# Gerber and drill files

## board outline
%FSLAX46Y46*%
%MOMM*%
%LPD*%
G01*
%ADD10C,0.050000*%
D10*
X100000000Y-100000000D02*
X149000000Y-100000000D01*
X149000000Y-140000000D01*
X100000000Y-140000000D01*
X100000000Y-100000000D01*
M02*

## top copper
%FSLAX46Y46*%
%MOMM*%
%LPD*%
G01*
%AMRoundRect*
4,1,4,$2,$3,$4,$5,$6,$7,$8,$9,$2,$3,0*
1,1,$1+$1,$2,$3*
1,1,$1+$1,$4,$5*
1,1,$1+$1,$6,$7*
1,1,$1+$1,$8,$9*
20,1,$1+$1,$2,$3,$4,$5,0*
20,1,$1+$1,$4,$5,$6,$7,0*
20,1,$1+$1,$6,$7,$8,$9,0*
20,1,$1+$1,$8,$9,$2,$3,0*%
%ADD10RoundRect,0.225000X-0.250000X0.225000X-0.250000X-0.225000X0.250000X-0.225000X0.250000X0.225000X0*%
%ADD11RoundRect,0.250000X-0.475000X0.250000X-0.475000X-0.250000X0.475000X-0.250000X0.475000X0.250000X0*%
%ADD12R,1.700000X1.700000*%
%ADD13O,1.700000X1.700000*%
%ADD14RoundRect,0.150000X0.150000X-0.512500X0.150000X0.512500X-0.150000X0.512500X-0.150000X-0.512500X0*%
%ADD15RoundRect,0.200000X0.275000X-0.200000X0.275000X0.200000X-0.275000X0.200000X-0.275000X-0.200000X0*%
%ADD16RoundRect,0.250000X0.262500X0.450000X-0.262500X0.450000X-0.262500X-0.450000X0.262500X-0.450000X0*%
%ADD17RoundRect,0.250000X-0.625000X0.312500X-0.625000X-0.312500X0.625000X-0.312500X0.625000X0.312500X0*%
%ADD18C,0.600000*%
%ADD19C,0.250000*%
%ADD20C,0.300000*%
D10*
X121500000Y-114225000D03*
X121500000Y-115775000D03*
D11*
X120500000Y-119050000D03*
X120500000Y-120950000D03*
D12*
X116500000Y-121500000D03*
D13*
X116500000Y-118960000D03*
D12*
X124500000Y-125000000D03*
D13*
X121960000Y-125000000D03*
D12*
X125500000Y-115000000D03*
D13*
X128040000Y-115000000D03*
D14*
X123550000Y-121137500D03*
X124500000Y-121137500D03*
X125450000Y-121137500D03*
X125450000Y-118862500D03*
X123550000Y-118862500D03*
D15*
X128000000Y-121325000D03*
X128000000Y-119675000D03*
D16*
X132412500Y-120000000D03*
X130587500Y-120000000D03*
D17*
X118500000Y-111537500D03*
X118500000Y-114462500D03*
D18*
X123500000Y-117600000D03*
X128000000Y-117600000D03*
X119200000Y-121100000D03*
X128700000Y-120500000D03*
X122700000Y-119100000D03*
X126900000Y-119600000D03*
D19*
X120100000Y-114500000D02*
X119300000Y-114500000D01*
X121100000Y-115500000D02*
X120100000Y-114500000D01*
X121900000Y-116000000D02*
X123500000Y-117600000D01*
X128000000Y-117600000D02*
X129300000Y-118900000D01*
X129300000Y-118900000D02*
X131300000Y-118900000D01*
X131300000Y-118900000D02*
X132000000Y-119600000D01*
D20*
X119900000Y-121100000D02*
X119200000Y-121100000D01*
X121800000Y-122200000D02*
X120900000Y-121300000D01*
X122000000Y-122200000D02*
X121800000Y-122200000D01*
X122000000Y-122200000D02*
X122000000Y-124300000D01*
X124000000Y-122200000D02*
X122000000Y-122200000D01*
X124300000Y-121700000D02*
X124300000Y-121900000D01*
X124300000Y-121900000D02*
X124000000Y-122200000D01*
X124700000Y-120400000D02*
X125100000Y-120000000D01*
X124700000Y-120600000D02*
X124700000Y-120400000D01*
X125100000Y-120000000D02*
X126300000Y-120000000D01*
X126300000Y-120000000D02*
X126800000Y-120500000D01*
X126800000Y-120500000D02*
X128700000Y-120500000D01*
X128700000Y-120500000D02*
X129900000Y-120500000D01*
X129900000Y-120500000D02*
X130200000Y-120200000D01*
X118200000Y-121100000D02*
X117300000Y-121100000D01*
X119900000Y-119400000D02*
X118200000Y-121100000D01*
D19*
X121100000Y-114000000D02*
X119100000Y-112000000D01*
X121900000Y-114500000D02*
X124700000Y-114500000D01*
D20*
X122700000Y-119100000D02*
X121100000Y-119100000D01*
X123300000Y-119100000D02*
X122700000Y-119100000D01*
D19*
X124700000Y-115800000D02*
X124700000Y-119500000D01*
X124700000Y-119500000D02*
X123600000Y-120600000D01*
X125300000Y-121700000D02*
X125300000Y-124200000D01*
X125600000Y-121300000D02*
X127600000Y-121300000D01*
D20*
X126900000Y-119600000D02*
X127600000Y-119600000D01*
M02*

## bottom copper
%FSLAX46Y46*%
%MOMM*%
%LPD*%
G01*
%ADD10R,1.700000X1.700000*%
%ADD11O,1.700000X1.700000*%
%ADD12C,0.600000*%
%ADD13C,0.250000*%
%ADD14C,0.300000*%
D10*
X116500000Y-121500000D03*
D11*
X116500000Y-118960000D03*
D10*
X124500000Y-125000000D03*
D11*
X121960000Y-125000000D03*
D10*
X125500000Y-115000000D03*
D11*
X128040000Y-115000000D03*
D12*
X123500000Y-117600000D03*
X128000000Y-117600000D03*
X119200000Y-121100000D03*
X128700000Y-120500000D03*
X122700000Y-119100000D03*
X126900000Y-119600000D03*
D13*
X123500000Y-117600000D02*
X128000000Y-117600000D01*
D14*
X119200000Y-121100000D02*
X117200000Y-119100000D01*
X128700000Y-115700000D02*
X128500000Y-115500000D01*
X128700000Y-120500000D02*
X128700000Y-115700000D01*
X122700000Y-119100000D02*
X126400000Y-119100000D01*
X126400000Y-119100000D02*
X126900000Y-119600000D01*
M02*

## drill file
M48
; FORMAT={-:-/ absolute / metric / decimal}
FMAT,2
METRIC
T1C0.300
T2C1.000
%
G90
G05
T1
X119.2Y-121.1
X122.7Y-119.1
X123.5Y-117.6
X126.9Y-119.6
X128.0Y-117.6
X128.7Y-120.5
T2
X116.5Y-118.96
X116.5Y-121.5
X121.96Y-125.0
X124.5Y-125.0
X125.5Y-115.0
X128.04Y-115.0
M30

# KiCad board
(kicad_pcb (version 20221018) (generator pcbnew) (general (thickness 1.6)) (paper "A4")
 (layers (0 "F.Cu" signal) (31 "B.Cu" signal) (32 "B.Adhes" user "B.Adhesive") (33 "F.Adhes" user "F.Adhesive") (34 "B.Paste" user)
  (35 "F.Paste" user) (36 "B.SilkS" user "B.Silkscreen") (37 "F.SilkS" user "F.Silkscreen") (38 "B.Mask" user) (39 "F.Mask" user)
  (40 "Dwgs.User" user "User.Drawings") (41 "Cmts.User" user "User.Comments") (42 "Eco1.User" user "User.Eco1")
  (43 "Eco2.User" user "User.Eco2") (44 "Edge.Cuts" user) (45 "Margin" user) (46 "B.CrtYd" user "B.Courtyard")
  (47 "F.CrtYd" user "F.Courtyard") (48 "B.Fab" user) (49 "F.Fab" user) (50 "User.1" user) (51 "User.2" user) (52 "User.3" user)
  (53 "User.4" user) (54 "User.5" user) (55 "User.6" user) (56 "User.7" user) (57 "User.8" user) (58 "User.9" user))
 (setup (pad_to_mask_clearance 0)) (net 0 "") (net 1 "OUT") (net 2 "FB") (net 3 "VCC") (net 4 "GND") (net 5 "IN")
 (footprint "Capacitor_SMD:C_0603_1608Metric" (layer "F.Cu") (at 121.5 115 -90)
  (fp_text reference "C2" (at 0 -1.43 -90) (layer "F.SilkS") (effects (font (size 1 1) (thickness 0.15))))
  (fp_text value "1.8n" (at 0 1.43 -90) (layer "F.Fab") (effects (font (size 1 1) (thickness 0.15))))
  (pad "1" smd roundrect (at -0.775 0 270) (size 0.9 0.95) (layers "F.Cu" "F.Paste" "F.Mask") (roundrect_rratio 0.25) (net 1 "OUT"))
  (pad "2" smd roundrect (at 0.775 0 270) (size 0.9 0.95) (layers "F.Cu" "F.Paste" "F.Mask") (roundrect_rratio 0.25) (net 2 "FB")))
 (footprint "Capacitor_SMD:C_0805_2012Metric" (layer "F.Cu") (at 120.5 120 -90)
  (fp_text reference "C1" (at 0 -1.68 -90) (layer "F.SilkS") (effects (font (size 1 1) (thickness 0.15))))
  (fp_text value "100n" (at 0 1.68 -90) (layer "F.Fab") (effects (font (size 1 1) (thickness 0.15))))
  (pad "1" smd roundrect (at -0.95 0 270) (size 1 1.45) (layers "F.Cu" "F.Paste" "F.Mask") (roundrect_rratio 0.25) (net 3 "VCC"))
  (pad "2" smd roundrect (at 0.95 0 270) (size 1 1.45) (layers "F.Cu" "F.Paste" "F.Mask") (roundrect_rratio 0.25) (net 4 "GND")))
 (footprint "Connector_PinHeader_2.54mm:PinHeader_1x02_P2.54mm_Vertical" (layer "F.Cu") (at 116.5 121.5 180)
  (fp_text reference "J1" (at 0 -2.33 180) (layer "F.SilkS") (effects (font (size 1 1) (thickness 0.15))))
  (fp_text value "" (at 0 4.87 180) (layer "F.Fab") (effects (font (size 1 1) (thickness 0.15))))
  (pad "1" thru_hole rect (at 0 0 180) (size 1.7 1.7) (drill 1) (layers "*.Cu" "*.Mask") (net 3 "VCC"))
  (pad "2" thru_hole oval (at 0 2.54 180) (size 1.7 1.7) (drill 1) (layers "*.Cu" "*.Mask") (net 4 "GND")))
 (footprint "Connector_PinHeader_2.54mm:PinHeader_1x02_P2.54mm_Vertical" (layer "F.Cu") (at 124.5 125 -90)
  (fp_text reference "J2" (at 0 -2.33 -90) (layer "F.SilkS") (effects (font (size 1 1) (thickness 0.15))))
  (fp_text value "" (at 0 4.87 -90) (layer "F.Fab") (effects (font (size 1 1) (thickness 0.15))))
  (pad "1" thru_hole rect (at 0 0 270) (size 1.7 1.7) (drill 1) (layers "*.Cu" "*.Mask") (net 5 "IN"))
  (pad "2" thru_hole oval (at 0 2.54 270) (size 1.7 1.7) (drill 1) (layers "*.Cu" "*.Mask") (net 4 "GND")))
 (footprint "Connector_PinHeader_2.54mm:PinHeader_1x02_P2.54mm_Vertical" (layer "F.Cu") (at 125.5 115 90)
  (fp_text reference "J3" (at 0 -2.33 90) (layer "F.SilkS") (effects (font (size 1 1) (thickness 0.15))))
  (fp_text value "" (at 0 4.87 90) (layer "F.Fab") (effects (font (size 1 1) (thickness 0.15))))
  (pad "1" thru_hole rect (at 0 0 90) (size 1.7 1.7) (drill 1) (layers "*.Cu" "*.Mask") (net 1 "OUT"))
  (pad "2" thru_hole oval (at 0 2.54 90) (size 1.7 1.7) (drill 1) (layers "*.Cu" "*.Mask") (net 4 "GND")))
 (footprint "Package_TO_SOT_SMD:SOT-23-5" (layer "F.Cu") (at 124.5 120 90)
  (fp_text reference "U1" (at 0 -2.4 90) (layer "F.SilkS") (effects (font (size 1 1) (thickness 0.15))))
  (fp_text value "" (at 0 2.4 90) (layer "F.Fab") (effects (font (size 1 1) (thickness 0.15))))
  (pad "1" smd roundrect (at -1.1375 -0.95 90) (size 1.325 0.6) (layers "F.Cu" "F.Paste" "F.Mask") (roundrect_rratio 0.25) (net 1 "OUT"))
  (pad "2" smd roundrect (at -1.1375 0 90) (size 1.325 0.6) (layers "F.Cu" "F.Paste" "F.Mask") (roundrect_rratio 0.25) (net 4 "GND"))
  (pad "3" smd roundrect (at -1.1375 0.95 90) (size 1.325 0.6) (layers "F.Cu" "F.Paste" "F.Mask") (roundrect_rratio 0.25) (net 5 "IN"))
  (pad "4" smd roundrect (at 1.1375 0.95 90) (size 1.325 0.6) (layers "F.Cu" "F.Paste" "F.Mask") (roundrect_rratio 0.25))
  (pad "5" smd roundrect (at 1.1375 -0.95 90) (size 1.325 0.6) (layers "F.Cu" "F.Paste" "F.Mask") (roundrect_rratio 0.25) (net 3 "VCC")))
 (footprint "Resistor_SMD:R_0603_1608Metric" (layer "F.Cu") (at 128 120.5 90)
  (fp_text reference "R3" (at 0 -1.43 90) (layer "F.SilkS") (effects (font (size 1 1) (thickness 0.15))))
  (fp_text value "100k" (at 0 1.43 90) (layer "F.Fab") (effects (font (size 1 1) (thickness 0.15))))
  (pad "1" smd roundrect (at -0.825 0 90) (size 0.8 0.95) (layers "F.Cu" "F.Paste" "F.Mask") (roundrect_rratio 0.25) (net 5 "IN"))
  (pad "2" smd roundrect (at 0.825 0 90) (size 0.8 0.95) (layers "F.Cu" "F.Paste" "F.Mask") (roundrect_rratio 0.25) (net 3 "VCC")))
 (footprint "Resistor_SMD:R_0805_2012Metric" (layer "F.Cu") (at 131.5 120 180)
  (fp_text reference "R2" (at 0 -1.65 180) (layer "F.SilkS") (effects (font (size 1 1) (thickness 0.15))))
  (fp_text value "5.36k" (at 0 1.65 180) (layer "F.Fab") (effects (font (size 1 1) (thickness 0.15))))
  (pad "1" smd roundrect (at -0.9125 0 180) (size 1.025 1.4) (layers "F.Cu" "F.Paste" "F.Mask") (roundrect_rratio 0.243902) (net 2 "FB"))
  (pad "2" smd roundrect (at 0.9125 0 180) (size 1.025 1.4) (layers "F.Cu" "F.Paste" "F.Mask") (roundrect_rratio 0.243902) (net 4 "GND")))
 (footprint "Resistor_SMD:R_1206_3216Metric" (layer "F.Cu") (at 118.5 113 -90)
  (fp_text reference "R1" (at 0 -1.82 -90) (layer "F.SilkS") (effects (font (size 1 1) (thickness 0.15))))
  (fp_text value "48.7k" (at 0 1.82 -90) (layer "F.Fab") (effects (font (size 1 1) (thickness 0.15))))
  (pad "1" smd roundrect (at -1.4625 0 270) (size 1.125 1.75) (layers "F.Cu" "F.Paste" "F.Mask") (roundrect_rratio 0.222222) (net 1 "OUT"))
  (pad "2" smd roundrect (at 1.4625 0 270) (size 1.125 1.75) (layers "F.Cu" "F.Paste" "F.Mask") (roundrect_rratio 0.222222) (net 2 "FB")))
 (gr_rect (start 100 100) (end 149 140) (stroke (width 0.05) (type default)) (fill none) (layer "Edge.Cuts"))
 (segment (start 120.1 114.5) (end 119.3 114.5) (width 0.25) (layer "F.Cu") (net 2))
 (segment (start 121.1 115.5) (end 120.1 114.5) (width 0.25) (layer "F.Cu") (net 2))
 (segment (start 121.9 116) (end 123.5 117.6) (width 0.25) (layer "F.Cu") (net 2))
 (segment (start 128 117.6) (end 129.3 118.9) (width 0.25) (layer "F.Cu") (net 2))
 (segment (start 129.3 118.9) (end 131.3 118.9) (width 0.25) (layer "F.Cu") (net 2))
 (segment (start 131.3 118.9) (end 132 119.6) (width 0.25) (layer "F.Cu") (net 2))
 (via (at 123.5 117.6) (size 0.6) (drill 0.3) (layers "F.Cu" "B.Cu") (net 2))
 (via (at 128 117.6) (size 0.6) (drill 0.3) (layers "F.Cu" "B.Cu") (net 2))
 (segment (start 119.9 121.1) (end 119.2 121.1) (width 0.3) (layer "F.Cu") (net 4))
 (segment (start 121.8 122.2) (end 120.9 121.3) (width 0.3) (layer "F.Cu") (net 4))
 (segment (start 122 122.2) (end 121.8 122.2) (width 0.3) (layer "F.Cu") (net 4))
 (segment (start 122 122.2) (end 122 124.3) (width 0.3) (layer "F.Cu") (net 4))
 (segment (start 123.5 117.6) (end 128 117.6) (width 0.25) (layer "B.Cu") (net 2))
 (segment (start 124 122.2) (end 122 122.2) (width 0.3) (layer "F.Cu") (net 4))
 (segment (start 124.3 121.7) (end 124.3 121.9) (width 0.3) (layer "F.Cu") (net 4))
 (segment (start 124.3 121.9) (end 124 122.2) (width 0.3) (layer "F.Cu") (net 4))
 (segment (start 124.7 120.4) (end 125.1 120) (width 0.3) (layer "F.Cu") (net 4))
 (segment (start 124.7 120.6) (end 124.7 120.4) (width 0.3) (layer "F.Cu") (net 4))
 (segment (start 125.1 120) (end 126.3 120) (width 0.3) (layer "F.Cu") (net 4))
 (segment (start 126.3 120) (end 126.8 120.5) (width 0.3) (layer "F.Cu") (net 4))
 (segment (start 126.8 120.5) (end 128.7 120.5) (width 0.3) (layer "F.Cu") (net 4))
 (segment (start 128.7 120.5) (end 129.9 120.5) (width 0.3) (layer "F.Cu") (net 4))
 (segment (start 129.9 120.5) (end 130.2 120.2) (width 0.3) (layer "F.Cu") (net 4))
 (via (at 119.2 121.1) (size 0.6) (drill 0.3) (layers "F.Cu" "B.Cu") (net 4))
 (via (at 128.7 120.5) (size 0.6) (drill 0.3) (layers "F.Cu" "B.Cu") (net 4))
 (segment (start 118.2 121.1) (end 117.3 121.1) (width 0.3) (layer "F.Cu") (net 3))
 (segment (start 119.2 121.1) (end 117.2 119.1) (width 0.3) (layer "B.Cu") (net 4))
 (segment (start 119.9 119.4) (end 118.2 121.1) (width 0.3) (layer "F.Cu") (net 3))
 (segment (start 121.1 114) (end 119.1 112) (width 0.25) (layer "F.Cu") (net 1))
 (segment (start 121.9 114.5) (end 124.7 114.5) (width 0.25) (layer "F.Cu") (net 1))
 (segment (start 122.7 119.1) (end 121.1 119.1) (width 0.3) (layer "F.Cu") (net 3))
 (segment (start 123.3 119.1) (end 122.7 119.1) (width 0.3) (layer "F.Cu") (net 3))
 (segment (start 124.7 115.8) (end 124.7 119.5) (width 0.25) (layer "F.Cu") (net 1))
 (segment (start 124.7 119.5) (end 123.6 120.6) (width 0.25) (layer "F.Cu") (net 1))
 (segment (start 125.3 121.7) (end 125.3 124.2) (width 0.25) (layer "F.Cu") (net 5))
 (segment (start 125.6 121.3) (end 127.6 121.3) (width 0.25) (layer "F.Cu") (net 5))
 (segment (start 126.9 119.6) (end 127.6 119.6) (width 0.3) (layer "F.Cu") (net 3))
 (segment (start 128.7 115.7) (end 128.5 115.5) (width 0.3) (layer "B.Cu") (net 4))
 (segment (start 128.7 120.5) (end 128.7 115.7) (width 0.3) (layer "B.Cu") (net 4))
 (via (at 122.7 119.1) (size 0.6) (drill 0.3) (layers "F.Cu" "B.Cu") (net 3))
 (via (at 126.9 119.6) (size 0.6) (drill 0.3) (layers "F.Cu" "B.Cu") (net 3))
 (segment (start 122.7 119.1) (end 126.4 119.1) (width 0.3) (layer "B.Cu") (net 3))
 (segment (start 126.4 119.1) (end 126.9 119.6) (width 0.3) (layer "B.Cu") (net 3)))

